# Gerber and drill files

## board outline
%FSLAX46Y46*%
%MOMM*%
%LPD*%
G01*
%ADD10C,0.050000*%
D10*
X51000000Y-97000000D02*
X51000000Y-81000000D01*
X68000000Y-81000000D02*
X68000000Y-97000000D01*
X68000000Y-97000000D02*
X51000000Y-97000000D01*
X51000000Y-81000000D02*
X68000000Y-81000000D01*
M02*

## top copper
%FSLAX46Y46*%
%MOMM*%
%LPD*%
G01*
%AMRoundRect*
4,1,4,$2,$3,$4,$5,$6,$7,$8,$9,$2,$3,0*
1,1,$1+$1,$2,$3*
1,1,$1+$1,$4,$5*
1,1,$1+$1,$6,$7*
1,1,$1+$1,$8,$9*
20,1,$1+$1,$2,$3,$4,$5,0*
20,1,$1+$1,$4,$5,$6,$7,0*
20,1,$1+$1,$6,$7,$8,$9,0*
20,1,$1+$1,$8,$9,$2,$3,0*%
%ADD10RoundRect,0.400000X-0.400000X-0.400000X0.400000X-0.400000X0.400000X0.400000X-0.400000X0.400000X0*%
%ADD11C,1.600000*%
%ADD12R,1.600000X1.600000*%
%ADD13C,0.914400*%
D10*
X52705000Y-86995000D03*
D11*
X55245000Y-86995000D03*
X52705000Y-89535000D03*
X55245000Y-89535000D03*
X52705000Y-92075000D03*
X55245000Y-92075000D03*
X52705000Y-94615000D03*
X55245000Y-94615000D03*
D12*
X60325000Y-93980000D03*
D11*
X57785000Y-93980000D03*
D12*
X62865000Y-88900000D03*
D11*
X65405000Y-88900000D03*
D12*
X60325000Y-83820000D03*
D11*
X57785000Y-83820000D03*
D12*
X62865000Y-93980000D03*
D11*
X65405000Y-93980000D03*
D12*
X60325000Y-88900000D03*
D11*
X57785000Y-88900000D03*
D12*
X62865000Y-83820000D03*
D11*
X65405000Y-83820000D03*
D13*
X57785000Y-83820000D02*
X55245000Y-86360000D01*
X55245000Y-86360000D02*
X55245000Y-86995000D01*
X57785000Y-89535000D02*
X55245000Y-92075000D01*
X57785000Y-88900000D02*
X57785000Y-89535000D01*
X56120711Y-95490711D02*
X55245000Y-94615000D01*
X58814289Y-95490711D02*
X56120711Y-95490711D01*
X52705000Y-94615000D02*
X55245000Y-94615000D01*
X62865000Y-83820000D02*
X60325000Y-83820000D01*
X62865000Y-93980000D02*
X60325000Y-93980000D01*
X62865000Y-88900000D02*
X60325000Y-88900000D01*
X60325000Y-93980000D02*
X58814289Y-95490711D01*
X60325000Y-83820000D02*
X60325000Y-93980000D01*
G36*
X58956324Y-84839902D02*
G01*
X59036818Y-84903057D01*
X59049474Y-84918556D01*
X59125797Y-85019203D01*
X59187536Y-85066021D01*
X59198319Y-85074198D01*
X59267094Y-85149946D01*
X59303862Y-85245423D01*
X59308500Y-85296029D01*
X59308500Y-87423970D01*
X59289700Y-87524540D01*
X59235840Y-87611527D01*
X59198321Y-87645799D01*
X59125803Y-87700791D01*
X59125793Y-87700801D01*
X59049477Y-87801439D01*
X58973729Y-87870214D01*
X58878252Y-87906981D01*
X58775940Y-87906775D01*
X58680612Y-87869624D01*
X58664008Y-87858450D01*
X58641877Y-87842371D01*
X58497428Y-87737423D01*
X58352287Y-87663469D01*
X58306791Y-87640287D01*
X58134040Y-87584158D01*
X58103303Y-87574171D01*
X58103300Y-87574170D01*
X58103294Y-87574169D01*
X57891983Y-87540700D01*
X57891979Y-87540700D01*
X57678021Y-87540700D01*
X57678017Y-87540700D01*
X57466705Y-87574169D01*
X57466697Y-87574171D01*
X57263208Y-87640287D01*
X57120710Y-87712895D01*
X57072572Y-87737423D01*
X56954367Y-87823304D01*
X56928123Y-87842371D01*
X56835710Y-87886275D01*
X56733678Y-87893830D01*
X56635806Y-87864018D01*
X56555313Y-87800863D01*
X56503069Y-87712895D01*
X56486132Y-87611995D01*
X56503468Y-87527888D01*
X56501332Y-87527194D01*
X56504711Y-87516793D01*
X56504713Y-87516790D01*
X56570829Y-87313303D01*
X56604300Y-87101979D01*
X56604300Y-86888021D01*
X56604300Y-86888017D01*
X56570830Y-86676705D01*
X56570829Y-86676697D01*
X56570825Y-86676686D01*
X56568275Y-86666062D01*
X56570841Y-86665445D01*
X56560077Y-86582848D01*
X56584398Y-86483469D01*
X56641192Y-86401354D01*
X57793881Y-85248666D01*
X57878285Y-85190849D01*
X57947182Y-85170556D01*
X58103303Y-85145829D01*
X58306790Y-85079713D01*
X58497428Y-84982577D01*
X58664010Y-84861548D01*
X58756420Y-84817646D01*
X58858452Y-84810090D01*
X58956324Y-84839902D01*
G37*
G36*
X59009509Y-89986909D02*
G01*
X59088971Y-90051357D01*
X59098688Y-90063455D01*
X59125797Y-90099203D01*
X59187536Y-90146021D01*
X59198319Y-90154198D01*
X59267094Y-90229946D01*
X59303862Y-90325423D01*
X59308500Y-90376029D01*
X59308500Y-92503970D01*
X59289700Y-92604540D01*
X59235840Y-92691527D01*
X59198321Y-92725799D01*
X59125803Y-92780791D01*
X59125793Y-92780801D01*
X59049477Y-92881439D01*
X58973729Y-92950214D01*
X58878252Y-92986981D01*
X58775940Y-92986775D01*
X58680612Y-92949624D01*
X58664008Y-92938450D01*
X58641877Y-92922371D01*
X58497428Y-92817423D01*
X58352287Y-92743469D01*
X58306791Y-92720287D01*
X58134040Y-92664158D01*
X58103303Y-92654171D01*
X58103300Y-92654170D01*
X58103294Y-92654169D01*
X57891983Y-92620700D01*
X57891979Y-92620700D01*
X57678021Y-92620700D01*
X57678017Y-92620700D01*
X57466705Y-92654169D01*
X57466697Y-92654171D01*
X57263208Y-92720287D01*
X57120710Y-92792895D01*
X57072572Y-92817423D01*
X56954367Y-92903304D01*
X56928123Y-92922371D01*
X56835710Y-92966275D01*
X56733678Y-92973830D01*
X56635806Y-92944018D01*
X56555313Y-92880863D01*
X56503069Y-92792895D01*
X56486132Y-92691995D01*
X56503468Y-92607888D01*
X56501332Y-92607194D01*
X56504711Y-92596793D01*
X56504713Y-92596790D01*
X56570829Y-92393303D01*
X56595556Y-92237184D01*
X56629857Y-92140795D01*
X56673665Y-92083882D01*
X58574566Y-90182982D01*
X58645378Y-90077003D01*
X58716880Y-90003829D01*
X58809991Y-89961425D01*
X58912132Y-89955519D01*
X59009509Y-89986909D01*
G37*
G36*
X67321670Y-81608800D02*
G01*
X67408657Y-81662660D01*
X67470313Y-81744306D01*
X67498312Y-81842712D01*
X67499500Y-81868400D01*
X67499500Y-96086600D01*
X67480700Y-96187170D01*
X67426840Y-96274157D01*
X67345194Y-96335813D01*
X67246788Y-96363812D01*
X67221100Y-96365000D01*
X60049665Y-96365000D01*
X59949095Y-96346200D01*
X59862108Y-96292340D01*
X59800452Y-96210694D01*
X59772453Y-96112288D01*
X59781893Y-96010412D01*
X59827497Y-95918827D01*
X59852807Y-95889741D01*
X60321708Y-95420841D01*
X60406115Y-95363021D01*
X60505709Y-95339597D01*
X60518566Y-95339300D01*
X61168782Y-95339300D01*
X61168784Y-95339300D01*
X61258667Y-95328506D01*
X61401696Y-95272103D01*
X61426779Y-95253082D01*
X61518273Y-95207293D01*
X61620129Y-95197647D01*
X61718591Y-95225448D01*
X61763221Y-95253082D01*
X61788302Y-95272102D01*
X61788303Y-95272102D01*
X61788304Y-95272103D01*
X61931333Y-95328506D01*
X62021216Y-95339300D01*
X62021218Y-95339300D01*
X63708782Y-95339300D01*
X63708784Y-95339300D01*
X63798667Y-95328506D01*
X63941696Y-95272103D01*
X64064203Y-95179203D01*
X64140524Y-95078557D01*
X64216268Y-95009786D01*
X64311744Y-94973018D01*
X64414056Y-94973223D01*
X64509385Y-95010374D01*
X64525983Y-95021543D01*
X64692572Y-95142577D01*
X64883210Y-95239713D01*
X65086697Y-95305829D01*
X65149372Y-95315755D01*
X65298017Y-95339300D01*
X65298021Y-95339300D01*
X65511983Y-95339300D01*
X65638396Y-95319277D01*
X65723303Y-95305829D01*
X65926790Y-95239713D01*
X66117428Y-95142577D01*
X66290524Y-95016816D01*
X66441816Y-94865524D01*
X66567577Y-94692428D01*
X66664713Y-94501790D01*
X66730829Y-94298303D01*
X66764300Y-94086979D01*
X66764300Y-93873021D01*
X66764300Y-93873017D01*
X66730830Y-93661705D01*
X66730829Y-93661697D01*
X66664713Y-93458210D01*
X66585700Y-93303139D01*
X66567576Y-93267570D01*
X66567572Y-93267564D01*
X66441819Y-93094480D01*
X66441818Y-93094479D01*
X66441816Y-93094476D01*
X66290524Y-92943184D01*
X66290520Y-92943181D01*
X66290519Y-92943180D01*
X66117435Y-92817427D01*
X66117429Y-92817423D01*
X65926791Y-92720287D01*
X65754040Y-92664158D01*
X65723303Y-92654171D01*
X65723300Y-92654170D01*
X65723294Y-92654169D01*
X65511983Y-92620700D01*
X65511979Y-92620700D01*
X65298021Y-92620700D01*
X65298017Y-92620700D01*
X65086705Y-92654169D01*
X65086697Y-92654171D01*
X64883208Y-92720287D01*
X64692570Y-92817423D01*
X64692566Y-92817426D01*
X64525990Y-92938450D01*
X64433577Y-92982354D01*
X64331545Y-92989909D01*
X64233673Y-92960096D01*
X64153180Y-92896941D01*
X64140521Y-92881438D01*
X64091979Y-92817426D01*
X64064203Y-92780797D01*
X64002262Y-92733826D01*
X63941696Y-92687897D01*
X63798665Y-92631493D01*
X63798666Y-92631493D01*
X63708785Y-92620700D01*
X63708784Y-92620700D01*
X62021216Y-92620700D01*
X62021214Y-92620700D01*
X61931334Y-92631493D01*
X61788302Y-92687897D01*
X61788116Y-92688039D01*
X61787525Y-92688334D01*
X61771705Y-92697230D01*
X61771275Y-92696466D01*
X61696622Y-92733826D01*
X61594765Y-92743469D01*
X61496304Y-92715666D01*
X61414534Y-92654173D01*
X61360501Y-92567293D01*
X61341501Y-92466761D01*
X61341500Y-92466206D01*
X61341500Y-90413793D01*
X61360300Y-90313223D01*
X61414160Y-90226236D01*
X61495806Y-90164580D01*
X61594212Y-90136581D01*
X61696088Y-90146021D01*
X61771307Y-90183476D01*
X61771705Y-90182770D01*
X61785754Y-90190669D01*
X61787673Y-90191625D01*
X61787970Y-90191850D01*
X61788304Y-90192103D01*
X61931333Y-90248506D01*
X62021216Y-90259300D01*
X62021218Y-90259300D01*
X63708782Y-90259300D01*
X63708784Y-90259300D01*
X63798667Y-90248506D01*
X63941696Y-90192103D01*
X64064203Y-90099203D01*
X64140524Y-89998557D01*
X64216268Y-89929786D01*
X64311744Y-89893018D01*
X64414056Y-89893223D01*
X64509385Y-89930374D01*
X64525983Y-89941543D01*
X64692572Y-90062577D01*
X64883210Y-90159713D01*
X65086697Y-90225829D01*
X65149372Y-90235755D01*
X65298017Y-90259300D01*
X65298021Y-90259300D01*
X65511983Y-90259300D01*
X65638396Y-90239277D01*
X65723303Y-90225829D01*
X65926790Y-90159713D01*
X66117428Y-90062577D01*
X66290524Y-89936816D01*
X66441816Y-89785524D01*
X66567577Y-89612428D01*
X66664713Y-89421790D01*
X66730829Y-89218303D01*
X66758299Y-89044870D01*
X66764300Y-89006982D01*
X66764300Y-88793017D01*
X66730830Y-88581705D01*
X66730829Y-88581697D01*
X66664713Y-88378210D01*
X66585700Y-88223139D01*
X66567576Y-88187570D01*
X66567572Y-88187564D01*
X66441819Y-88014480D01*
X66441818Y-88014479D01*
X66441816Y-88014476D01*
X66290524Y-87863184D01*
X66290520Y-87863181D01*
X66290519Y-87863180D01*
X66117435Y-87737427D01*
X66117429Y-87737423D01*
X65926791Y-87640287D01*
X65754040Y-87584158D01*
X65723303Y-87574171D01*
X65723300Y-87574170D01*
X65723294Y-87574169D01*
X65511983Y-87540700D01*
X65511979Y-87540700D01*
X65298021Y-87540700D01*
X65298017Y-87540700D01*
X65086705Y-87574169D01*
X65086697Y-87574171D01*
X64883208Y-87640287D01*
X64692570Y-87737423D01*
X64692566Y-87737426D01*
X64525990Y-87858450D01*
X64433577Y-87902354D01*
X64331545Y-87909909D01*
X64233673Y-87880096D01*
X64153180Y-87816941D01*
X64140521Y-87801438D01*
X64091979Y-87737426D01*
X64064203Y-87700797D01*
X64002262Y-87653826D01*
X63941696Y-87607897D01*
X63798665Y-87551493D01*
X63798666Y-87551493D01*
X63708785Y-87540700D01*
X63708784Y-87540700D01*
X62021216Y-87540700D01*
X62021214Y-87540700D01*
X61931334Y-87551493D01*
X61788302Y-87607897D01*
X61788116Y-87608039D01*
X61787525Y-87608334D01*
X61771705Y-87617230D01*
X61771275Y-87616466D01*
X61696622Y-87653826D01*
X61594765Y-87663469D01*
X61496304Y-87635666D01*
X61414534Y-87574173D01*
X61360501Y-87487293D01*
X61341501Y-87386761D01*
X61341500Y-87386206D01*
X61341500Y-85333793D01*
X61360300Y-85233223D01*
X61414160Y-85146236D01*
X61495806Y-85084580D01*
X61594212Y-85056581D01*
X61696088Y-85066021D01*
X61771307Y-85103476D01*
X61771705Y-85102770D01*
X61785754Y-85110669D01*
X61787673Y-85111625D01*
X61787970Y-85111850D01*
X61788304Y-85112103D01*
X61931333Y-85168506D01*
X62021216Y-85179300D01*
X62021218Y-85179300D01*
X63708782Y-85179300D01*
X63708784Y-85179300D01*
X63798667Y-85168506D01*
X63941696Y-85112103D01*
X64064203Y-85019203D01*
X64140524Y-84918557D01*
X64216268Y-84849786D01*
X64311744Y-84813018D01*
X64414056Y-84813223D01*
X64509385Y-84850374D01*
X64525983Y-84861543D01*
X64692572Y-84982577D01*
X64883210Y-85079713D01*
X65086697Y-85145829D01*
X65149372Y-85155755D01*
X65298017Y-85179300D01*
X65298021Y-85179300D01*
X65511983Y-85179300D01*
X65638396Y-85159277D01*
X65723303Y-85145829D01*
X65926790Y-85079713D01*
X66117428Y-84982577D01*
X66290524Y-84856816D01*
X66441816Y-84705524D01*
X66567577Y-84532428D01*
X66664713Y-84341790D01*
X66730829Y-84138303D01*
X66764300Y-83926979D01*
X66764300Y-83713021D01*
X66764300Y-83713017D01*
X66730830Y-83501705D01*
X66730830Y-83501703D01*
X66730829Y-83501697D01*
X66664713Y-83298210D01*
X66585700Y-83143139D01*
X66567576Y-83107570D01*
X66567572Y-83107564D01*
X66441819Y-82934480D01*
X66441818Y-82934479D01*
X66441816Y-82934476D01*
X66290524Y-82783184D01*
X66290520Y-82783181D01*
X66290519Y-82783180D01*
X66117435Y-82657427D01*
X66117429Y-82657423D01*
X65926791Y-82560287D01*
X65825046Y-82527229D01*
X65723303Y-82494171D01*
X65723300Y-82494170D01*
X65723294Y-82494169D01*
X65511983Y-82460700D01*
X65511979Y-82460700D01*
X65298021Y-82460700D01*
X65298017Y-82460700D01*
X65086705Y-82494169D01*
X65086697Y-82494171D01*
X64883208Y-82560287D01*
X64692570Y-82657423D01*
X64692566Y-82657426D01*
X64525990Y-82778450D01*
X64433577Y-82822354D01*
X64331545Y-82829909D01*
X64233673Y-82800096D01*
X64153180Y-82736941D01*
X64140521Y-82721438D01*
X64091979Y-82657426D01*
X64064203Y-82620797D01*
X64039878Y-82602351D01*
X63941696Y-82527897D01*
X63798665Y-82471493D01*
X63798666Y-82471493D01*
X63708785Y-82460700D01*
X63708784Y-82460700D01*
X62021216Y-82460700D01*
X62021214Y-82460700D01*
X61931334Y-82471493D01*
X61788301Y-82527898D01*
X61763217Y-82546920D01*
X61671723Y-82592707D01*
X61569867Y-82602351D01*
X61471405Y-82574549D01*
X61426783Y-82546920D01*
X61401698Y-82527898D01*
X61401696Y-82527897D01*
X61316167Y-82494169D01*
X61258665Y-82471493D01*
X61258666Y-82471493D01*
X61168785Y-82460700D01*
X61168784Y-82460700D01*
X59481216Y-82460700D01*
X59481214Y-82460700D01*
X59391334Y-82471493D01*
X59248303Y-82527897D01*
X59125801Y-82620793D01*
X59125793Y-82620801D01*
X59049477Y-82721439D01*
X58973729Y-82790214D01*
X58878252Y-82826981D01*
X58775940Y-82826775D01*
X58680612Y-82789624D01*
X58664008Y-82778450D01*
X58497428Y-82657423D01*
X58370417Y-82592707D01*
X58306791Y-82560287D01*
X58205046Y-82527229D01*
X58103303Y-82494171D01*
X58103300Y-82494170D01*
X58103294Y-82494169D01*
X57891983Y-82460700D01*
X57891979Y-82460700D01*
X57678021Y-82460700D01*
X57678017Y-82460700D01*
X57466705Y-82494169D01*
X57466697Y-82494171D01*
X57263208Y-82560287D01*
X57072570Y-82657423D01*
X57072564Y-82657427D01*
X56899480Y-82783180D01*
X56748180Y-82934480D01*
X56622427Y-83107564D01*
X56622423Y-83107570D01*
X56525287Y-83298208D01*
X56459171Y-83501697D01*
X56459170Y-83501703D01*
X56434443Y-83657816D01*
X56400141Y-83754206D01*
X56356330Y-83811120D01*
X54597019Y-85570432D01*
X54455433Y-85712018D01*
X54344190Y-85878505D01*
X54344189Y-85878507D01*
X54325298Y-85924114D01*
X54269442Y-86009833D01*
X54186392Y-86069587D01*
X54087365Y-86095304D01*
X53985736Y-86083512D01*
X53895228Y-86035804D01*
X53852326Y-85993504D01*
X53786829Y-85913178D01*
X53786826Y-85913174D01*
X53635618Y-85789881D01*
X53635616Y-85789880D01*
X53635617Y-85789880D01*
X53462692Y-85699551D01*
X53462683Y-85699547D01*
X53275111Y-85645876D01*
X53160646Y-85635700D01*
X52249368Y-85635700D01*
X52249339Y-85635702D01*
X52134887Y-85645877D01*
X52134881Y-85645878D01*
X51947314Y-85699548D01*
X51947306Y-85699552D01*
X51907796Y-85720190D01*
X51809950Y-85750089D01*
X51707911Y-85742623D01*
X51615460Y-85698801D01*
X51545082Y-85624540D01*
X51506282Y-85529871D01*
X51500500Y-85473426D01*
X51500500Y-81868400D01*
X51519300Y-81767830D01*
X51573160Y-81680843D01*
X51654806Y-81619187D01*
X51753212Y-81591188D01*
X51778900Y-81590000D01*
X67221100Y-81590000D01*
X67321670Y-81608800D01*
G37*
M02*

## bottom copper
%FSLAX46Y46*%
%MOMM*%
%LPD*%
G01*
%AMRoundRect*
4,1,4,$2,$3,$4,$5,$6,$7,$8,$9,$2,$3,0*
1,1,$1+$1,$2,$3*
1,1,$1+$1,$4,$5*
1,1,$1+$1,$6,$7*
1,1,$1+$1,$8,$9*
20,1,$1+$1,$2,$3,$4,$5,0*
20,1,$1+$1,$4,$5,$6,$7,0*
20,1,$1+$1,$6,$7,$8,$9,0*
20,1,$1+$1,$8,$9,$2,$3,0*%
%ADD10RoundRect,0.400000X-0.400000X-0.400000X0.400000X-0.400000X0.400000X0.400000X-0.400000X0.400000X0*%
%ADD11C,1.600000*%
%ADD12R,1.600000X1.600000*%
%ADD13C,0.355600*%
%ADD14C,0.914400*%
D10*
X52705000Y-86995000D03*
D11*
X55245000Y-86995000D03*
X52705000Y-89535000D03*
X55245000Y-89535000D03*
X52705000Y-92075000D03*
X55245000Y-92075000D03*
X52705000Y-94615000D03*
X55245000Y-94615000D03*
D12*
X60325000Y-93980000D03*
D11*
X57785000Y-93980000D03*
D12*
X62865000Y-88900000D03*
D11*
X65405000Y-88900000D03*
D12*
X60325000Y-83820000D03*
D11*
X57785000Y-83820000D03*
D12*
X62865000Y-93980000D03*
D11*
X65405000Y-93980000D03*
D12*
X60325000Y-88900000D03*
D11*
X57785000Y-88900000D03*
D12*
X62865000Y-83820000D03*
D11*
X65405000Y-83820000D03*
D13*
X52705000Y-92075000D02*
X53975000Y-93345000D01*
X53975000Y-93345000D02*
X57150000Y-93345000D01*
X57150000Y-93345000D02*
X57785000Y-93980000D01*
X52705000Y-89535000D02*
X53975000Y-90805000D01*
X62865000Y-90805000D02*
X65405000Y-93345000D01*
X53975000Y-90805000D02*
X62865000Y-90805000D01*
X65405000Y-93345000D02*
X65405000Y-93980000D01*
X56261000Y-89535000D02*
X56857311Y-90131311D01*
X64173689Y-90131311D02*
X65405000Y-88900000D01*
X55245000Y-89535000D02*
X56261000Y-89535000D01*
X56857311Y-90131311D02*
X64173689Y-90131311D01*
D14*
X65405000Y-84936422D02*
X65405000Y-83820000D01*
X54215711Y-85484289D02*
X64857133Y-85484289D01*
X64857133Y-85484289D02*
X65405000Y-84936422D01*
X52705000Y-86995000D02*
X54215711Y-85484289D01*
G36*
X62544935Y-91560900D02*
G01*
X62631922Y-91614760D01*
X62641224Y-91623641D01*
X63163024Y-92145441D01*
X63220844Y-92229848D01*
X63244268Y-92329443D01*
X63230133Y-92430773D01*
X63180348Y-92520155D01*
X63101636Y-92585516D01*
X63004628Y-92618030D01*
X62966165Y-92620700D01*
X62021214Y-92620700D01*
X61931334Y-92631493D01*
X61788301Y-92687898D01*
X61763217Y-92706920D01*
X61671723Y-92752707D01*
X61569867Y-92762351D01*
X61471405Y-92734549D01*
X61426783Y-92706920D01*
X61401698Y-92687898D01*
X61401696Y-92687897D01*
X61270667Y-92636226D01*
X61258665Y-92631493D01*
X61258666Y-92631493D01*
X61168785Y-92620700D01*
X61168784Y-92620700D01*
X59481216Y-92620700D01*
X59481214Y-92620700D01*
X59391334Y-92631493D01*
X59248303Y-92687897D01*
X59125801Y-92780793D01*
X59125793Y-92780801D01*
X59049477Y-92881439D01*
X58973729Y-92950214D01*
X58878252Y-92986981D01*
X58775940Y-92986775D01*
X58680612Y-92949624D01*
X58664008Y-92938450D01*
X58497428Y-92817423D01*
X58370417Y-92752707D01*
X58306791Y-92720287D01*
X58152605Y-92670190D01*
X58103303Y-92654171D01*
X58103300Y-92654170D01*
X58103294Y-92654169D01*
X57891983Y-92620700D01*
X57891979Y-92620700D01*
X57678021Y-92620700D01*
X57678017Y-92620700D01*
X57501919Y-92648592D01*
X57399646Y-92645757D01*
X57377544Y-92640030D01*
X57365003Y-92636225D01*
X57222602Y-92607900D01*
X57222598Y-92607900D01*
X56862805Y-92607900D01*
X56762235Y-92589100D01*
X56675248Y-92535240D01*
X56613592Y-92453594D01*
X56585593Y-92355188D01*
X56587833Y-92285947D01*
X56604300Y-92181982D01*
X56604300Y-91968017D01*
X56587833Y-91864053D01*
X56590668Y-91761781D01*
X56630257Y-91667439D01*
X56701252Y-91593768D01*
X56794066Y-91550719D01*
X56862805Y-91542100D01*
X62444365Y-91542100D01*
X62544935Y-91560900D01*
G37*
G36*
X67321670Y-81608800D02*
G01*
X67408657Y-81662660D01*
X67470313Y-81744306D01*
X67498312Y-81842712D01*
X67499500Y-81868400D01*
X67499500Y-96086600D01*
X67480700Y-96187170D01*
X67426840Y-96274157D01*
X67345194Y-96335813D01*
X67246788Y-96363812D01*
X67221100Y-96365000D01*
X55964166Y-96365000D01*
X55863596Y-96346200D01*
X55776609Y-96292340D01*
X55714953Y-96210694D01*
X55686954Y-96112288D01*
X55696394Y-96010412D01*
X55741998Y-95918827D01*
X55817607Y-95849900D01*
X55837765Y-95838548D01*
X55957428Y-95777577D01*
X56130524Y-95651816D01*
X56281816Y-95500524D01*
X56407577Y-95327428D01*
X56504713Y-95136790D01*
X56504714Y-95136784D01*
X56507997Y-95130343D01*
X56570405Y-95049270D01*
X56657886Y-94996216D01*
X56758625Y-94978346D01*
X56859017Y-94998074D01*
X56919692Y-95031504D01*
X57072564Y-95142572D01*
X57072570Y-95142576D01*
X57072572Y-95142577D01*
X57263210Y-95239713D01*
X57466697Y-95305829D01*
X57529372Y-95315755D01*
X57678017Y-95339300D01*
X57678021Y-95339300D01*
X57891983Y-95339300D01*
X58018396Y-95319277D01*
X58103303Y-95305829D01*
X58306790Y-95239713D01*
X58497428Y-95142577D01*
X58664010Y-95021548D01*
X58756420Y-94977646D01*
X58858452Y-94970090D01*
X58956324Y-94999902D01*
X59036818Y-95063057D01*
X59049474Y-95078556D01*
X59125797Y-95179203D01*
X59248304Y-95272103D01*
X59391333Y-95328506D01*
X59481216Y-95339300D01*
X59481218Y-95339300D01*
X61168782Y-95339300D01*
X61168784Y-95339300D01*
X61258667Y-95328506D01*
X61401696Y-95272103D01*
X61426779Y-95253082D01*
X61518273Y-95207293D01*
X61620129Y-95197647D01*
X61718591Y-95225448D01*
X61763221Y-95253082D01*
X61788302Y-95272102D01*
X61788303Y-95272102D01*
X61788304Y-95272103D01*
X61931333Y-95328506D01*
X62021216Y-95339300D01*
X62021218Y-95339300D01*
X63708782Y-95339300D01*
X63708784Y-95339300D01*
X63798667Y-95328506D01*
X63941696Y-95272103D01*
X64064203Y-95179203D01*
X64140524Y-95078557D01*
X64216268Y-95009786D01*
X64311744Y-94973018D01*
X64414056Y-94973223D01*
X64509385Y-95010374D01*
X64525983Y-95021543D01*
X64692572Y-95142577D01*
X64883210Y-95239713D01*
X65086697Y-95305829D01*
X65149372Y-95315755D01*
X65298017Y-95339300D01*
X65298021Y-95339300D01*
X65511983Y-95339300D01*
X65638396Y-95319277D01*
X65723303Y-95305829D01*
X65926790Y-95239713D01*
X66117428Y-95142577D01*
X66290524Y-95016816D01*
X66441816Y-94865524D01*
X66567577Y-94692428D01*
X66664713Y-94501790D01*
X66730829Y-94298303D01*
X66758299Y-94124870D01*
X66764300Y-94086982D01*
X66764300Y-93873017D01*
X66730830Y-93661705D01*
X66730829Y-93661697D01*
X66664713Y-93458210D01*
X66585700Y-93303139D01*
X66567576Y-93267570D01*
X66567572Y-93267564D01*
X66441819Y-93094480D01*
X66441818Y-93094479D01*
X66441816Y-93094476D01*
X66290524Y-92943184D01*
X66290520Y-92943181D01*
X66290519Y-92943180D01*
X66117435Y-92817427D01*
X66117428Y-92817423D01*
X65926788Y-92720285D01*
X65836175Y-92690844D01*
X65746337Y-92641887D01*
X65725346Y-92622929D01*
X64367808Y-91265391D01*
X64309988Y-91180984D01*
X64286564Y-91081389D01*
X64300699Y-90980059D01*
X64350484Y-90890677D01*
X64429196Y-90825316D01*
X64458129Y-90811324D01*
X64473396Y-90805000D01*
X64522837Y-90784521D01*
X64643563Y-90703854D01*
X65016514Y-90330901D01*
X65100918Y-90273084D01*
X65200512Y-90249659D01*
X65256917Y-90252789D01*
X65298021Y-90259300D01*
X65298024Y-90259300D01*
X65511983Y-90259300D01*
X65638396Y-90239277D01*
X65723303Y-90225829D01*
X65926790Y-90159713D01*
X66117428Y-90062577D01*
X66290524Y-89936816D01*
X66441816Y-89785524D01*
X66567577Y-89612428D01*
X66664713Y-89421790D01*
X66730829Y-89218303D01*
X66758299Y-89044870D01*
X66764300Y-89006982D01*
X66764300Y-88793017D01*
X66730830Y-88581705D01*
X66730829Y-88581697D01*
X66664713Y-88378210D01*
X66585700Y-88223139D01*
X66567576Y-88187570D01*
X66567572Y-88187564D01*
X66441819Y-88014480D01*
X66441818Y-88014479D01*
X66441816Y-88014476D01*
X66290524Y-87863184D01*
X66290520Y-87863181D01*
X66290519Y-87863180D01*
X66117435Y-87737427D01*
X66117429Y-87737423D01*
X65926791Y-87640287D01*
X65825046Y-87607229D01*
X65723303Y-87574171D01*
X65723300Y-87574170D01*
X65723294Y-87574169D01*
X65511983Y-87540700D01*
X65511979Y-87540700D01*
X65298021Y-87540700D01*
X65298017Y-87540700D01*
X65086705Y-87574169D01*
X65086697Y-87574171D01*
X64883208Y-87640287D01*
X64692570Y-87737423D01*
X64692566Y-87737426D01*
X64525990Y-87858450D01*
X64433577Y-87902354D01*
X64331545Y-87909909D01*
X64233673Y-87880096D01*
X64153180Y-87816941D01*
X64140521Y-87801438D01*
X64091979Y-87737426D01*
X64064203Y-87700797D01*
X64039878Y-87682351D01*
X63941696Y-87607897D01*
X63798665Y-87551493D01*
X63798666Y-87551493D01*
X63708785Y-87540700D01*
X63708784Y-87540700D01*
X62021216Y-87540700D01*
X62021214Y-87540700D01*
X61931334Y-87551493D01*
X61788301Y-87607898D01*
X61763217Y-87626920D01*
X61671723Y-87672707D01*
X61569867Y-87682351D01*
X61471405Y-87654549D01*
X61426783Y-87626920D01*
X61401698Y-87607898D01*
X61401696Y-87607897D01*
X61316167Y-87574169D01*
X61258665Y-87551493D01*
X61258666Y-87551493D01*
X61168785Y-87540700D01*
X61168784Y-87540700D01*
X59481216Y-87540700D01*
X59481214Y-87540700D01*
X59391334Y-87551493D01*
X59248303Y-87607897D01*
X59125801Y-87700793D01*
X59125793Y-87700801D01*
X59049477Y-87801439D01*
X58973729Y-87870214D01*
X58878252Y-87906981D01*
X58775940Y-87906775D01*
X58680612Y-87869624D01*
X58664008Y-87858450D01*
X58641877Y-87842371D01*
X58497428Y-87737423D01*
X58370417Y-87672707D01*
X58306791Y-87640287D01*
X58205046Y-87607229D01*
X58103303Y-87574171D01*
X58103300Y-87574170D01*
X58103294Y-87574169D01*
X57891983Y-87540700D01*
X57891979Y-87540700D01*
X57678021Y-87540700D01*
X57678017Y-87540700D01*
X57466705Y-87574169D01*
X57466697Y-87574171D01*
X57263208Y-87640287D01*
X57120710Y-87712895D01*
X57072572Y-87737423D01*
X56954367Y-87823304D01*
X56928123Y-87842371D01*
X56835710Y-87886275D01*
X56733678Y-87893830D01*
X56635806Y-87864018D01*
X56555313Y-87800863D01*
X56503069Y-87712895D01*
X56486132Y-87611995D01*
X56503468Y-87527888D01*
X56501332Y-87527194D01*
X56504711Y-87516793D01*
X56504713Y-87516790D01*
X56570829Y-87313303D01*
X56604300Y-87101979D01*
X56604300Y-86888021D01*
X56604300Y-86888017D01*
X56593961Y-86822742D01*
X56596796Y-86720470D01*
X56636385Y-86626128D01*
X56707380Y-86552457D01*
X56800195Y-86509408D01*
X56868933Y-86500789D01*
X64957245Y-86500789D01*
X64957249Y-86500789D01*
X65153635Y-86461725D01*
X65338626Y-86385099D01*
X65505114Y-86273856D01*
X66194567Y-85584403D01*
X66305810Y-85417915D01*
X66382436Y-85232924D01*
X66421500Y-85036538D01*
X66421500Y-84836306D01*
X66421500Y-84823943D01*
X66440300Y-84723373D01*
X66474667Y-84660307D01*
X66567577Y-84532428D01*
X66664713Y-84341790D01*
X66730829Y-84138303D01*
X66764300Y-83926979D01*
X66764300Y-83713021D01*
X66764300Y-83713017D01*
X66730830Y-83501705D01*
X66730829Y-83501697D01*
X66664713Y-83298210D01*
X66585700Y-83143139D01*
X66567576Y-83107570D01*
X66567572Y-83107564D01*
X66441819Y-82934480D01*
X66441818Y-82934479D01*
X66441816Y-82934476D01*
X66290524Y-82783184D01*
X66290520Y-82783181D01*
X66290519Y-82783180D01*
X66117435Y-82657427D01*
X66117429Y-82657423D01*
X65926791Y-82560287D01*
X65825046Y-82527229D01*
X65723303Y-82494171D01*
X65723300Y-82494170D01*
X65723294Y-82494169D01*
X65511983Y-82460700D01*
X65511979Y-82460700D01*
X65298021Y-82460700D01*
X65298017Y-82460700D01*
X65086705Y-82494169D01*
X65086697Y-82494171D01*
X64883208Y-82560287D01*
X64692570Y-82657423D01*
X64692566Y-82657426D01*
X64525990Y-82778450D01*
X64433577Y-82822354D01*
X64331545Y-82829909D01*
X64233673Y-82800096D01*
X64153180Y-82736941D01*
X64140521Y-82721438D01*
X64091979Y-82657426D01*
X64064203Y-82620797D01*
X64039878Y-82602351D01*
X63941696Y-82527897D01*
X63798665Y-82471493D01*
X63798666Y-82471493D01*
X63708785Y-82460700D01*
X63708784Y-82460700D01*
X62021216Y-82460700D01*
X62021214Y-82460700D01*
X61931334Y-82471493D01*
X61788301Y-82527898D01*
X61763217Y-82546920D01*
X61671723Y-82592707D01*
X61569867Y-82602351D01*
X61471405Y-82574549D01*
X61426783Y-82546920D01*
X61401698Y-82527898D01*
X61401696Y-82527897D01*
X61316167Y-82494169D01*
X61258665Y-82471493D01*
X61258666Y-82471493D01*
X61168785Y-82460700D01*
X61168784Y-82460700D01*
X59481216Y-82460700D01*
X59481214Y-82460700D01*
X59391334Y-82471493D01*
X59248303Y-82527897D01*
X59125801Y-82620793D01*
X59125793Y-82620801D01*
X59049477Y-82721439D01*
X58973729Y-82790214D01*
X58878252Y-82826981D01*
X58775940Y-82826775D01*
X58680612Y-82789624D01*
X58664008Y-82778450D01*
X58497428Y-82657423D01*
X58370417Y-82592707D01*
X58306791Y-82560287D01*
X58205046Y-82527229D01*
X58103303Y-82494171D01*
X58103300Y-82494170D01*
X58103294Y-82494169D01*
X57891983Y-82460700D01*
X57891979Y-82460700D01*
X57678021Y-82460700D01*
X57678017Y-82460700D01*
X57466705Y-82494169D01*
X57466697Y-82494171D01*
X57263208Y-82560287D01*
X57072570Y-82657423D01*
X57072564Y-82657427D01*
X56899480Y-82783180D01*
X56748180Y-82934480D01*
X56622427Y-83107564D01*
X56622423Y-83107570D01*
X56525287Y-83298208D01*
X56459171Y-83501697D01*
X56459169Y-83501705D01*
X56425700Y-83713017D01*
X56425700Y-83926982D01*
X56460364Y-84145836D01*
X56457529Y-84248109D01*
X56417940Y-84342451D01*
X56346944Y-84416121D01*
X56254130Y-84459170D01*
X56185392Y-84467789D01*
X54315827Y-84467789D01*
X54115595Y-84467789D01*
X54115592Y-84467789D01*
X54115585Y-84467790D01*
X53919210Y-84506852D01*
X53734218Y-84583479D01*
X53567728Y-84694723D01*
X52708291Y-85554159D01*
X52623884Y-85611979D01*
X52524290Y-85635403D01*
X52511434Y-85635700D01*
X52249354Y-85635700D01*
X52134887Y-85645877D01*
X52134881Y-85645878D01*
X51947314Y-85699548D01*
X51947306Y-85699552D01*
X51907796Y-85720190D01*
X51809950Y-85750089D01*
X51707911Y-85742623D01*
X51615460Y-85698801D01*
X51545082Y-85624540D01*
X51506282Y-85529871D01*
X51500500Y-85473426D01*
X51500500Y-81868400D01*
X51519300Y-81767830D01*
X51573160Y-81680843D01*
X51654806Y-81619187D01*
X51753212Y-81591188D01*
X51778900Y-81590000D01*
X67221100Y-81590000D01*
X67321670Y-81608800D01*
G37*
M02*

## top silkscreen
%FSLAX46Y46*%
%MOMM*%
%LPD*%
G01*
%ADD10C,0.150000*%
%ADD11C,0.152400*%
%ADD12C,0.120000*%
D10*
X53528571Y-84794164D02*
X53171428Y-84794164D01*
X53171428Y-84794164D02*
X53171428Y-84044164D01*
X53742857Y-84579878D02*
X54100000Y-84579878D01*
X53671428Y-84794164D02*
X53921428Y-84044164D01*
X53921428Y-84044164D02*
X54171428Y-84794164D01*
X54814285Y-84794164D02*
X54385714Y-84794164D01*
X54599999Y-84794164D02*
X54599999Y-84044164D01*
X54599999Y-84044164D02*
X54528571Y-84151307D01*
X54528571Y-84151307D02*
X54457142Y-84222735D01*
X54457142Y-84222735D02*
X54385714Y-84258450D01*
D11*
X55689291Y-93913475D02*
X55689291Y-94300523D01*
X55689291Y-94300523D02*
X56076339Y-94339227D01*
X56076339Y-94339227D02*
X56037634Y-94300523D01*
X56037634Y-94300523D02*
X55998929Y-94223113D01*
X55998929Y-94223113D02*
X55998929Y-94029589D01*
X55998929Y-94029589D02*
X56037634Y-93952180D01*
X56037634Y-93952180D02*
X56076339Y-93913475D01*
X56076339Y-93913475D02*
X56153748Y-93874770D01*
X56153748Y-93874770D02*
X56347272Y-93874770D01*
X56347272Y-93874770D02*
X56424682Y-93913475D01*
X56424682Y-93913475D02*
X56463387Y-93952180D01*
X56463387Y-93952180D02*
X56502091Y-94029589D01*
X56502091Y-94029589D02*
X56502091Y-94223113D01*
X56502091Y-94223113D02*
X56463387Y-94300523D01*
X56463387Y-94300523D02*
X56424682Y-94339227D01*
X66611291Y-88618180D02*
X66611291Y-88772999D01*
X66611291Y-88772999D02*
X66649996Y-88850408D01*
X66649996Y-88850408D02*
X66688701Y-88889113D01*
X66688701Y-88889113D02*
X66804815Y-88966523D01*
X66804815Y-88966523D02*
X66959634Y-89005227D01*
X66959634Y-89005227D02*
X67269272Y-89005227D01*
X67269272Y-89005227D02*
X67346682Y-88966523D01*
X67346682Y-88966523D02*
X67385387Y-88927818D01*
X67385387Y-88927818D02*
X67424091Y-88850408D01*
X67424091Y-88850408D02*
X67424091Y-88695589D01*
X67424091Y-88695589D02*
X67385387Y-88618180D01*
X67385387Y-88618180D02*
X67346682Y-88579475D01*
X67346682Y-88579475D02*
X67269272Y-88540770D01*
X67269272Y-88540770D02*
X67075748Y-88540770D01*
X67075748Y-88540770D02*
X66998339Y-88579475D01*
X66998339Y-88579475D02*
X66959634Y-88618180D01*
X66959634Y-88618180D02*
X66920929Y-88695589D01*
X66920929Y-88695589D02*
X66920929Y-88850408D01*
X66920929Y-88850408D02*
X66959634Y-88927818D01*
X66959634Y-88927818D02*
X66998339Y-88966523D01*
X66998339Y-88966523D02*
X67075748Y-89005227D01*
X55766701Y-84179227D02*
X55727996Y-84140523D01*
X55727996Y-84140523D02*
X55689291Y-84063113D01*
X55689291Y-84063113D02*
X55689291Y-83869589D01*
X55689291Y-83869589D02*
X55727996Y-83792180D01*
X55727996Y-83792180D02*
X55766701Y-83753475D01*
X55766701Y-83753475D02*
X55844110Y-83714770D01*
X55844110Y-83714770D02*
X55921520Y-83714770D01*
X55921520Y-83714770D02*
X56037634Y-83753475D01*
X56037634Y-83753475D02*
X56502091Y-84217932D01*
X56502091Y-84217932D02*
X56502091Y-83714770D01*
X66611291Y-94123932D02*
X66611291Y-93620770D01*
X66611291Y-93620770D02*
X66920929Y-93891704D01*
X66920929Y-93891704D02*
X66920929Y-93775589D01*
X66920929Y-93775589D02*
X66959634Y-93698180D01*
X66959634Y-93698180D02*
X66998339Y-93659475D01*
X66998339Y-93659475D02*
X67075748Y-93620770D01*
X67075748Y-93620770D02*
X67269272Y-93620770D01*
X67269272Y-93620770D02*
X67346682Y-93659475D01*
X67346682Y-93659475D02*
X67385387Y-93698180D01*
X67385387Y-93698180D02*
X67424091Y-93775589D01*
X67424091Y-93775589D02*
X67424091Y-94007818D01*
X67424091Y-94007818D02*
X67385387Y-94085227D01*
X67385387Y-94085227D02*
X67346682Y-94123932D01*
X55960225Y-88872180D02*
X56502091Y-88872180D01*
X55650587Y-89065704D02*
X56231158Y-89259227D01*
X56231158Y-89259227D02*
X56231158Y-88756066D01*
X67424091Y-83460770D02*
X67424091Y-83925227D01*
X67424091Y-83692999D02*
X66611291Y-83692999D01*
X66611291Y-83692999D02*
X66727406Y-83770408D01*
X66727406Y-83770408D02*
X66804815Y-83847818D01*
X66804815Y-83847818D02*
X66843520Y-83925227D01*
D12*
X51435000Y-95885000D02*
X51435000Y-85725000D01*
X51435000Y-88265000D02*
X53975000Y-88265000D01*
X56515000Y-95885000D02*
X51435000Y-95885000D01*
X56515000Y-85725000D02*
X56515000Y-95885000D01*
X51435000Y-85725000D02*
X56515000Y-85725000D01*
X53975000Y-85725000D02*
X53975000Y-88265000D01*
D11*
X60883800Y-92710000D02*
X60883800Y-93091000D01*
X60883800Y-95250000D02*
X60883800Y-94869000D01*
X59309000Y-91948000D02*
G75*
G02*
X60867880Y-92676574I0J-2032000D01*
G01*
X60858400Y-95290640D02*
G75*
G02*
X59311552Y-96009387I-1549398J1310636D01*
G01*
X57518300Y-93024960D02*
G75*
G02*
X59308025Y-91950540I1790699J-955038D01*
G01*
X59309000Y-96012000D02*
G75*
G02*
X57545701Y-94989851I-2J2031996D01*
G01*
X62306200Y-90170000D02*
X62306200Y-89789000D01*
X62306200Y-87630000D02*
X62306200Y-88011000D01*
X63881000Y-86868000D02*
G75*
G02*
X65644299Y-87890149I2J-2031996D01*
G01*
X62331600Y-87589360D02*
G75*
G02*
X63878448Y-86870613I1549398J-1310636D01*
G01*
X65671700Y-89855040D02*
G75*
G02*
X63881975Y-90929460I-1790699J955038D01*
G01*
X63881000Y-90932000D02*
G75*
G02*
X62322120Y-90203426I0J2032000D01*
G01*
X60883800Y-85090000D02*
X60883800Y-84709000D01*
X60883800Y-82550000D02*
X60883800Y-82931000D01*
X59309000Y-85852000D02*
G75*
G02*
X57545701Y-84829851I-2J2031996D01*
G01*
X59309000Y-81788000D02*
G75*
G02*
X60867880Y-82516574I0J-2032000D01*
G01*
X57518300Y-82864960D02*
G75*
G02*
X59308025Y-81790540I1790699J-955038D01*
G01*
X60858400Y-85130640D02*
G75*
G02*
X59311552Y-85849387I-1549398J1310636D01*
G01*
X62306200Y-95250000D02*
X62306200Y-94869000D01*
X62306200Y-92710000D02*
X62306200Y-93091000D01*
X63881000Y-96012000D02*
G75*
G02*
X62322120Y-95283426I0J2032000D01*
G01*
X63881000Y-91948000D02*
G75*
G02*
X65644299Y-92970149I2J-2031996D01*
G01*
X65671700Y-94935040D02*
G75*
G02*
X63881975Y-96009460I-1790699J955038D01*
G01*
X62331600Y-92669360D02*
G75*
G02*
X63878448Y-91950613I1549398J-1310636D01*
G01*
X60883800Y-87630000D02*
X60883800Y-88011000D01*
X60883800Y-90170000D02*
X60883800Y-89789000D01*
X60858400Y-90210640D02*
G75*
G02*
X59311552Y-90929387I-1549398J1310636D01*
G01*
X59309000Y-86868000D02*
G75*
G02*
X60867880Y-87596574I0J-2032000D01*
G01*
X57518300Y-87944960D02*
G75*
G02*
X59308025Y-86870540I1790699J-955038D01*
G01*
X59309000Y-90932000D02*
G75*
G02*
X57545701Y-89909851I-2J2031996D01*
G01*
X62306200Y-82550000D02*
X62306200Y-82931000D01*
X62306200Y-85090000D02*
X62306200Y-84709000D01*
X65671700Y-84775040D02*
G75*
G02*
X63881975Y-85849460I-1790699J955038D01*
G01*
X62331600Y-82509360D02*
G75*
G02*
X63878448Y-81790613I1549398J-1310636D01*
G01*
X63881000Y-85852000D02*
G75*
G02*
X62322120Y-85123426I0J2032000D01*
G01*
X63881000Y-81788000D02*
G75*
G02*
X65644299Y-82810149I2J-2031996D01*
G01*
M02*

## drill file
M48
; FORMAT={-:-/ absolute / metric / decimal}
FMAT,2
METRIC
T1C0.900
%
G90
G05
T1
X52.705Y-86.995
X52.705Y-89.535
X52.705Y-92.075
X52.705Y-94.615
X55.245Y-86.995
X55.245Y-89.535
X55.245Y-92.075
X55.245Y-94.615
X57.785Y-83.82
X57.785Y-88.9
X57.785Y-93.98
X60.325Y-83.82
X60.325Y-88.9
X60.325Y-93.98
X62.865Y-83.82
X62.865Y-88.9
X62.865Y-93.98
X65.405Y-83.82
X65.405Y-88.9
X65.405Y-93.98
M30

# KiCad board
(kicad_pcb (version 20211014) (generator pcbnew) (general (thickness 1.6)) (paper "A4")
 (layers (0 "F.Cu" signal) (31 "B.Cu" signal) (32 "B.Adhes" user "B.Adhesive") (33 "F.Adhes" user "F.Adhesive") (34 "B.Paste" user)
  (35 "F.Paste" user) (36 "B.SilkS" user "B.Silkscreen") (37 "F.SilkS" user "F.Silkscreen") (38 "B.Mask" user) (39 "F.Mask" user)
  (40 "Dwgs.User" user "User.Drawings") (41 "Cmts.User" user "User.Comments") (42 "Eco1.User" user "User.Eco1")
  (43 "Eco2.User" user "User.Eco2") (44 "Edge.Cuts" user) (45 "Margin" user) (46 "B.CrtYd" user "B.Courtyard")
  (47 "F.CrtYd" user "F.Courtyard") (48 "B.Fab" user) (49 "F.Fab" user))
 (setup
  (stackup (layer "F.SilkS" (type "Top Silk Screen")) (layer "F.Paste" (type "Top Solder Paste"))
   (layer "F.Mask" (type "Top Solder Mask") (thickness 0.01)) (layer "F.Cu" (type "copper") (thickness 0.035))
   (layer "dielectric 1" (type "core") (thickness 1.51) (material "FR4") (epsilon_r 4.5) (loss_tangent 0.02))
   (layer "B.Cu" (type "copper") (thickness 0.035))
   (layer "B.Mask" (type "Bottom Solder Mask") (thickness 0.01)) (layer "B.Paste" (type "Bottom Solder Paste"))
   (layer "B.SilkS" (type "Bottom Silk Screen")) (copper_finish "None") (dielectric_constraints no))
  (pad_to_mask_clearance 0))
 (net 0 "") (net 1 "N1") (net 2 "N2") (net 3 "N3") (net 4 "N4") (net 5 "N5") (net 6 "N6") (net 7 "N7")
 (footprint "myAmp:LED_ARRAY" (layer "F.Cu") (at 53.975 90.805)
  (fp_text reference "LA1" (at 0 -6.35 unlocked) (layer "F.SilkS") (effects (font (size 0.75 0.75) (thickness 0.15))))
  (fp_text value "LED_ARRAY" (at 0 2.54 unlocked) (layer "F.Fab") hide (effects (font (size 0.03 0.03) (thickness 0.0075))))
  (fp_line (start -2.54 5.08) (end -2.54 -5.08) (layer "F.SilkS") (width 0.12))
  (fp_line (start -2.54 -2.54) (end 0 -2.54) (layer "F.SilkS") (width 0.12))
  (fp_line (start 2.54 5.08) (end -2.54 5.08) (layer "F.SilkS") (width 0.12))
  (fp_line (start 2.54 -5.08) (end 2.54 5.08) (layer "F.SilkS") (width 0.12))
  (fp_line (start -2.54 -5.08) (end 2.54 -5.08) (layer "F.SilkS") (width 0.12))
  (fp_line (start 0 -5.08) (end 0 -2.54) (layer "F.SilkS") (width 0.12))
  (pad "1" thru_hole roundrect (at -1.27 -3.81) (size 1.6 1.6) (drill 0.9) (layers *.Cu *.Mask) (roundrect_rratio 0.25) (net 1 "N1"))
  (pad "2" thru_hole circle (at 1.27 -3.81) (size 1.6 1.6) (drill 0.9) (layers *.Cu *.Mask) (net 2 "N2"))
  (pad "3" thru_hole circle (at -1.27 -1.27) (size 1.6 1.6) (drill 0.9) (layers *.Cu *.Mask) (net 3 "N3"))
  (pad "4" thru_hole circle (at 1.27 -1.27) (size 1.6 1.6) (drill 0.9) (layers *.Cu *.Mask) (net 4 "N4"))
  (pad "5" thru_hole circle (at -1.27 1.27) (size 1.6 1.6) (drill 0.9) (layers *.Cu *.Mask) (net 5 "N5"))
  (pad "6" thru_hole circle (at 1.27 1.27) (size 1.6 1.6) (drill 0.9) (layers *.Cu *.Mask) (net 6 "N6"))
  (pad "7" thru_hole circle (at -1.27 3.81) (size 1.6 1.6) (drill 0.9) (layers *.Cu *.Mask) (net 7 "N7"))
  (pad "8" thru_hole circle (at 1.27 3.81) (size 1.6 1.6) (drill 0.9) (layers *.Cu *.Mask) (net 7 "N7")))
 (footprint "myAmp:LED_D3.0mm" (layer "F.Cu") (at 59.055 93.98)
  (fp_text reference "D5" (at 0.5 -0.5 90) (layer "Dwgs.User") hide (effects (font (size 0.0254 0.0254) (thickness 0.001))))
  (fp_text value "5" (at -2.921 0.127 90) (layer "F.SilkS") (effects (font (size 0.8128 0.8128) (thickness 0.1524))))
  (fp_line (start 1.8288 -1.27) (end 1.8288 -0.889) (layer "F.SilkS") (width 0.1524))
  (fp_line (start 1.8288 1.27) (end 1.8288 0.889) (layer "F.SilkS") (width 0.1524))
  (fp_arc (start 0.254 -2.032) (mid 1.114367 -1.840867) (end 1.81288 -1.303426) (layer "F.SilkS") (width 0.1524))
  (fp_arc (start 1.8034 1.31064) (mid 1.109154 1.840416) (end 0.256552 2.029387) (layer "F.SilkS") (width 0.1524))
  (fp_arc (start -1.5367 -0.95504) (mid -0.790567 -1.739997) (end 0.253025 -2.02946) (layer "F.SilkS") (width 0.1524))
  (fp_arc (start 0.254 2.032) (mid -0.76507 1.757988) (end -1.509299 1.009851) (layer "F.SilkS") (width 0.1524))
  (pad "1" thru_hole rect locked (at 1.27 0) (size 1.6 1.6) (drill 0.9) (layers *.Cu *.Mask) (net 7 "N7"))
  (pad "2" thru_hole circle locked (at -1.27 0) (size 1.6 1.6) (drill 0.9) (layers *.Cu *.Mask) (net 5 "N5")))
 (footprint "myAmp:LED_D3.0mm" (layer "F.Cu") (at 64.135 88.9 180)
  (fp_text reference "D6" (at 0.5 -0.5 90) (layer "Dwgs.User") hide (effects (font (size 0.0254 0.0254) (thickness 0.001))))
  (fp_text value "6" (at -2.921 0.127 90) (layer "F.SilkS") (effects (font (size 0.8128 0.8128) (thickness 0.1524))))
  (fp_line (start 1.8288 -1.27) (end 1.8288 -0.889) (layer "F.SilkS") (width 0.1524))
  (fp_line (start 1.8288 1.27) (end 1.8288 0.889) (layer "F.SilkS") (width 0.1524))
  (fp_arc (start 0.254 2.032) (mid -0.76507 1.757988) (end -1.509299 1.009851) (layer "F.SilkS") (width 0.1524))
  (fp_arc (start 1.8034 1.31064) (mid 1.109154 1.840416) (end 0.256552 2.029387) (layer "F.SilkS") (width 0.1524))
  (fp_arc (start -1.5367 -0.95504) (mid -0.790567 -1.739997) (end 0.253025 -2.02946) (layer "F.SilkS") (width 0.1524))
  (fp_arc (start 0.254 -2.032) (mid 1.114367 -1.840867) (end 1.81288 -1.303426) (layer "F.SilkS") (width 0.1524))
  (pad "1" thru_hole rect locked (at 1.27 0 180) (size 1.6 1.6) (drill 0.9) (layers *.Cu *.Mask) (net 7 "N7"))
  (pad "2" thru_hole circle locked (at -1.27 0 180) (size 1.6 1.6) (drill 0.9) (layers *.Cu *.Mask) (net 4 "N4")))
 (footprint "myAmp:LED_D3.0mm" (layer "F.Cu") (at 59.055 83.82)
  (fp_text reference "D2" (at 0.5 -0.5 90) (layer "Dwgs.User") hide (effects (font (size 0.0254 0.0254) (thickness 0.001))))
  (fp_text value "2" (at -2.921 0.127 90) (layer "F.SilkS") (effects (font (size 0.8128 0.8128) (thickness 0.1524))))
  (fp_line (start 1.8288 1.27) (end 1.8288 0.889) (layer "F.SilkS") (width 0.1524))
  (fp_line (start 1.8288 -1.27) (end 1.8288 -0.889) (layer "F.SilkS") (width 0.1524))
  (fp_arc (start 0.254 2.032) (mid -0.76507 1.757988) (end -1.509299 1.009851) (layer "F.SilkS") (width 0.1524))
  (fp_arc (start 0.254 -2.032) (mid 1.114367 -1.840867) (end 1.81288 -1.303426) (layer "F.SilkS") (width 0.1524))
  (fp_arc (start -1.5367 -0.95504) (mid -0.790567 -1.739997) (end 0.253025 -2.02946) (layer "F.SilkS") (width 0.1524))
  (fp_arc (start 1.8034 1.31064) (mid 1.109154 1.840416) (end 0.256552 2.029387) (layer "F.SilkS") (width 0.1524))
  (pad "1" thru_hole rect locked (at 1.27 0) (size 1.6 1.6) (drill 0.9) (layers *.Cu *.Mask) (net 7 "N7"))
  (pad "2" thru_hole circle locked (at -1.27 0) (size 1.6 1.6) (drill 0.9) (layers *.Cu *.Mask) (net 2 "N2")))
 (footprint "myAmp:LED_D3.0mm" (layer "F.Cu") (at 64.135 93.98 180)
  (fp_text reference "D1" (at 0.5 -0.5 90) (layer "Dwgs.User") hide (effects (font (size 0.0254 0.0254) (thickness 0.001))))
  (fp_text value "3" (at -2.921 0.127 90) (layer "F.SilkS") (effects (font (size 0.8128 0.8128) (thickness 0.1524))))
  (fp_line (start 1.8288 -1.27) (end 1.8288 -0.889) (layer "F.SilkS") (width 0.1524))
  (fp_line (start 1.8288 1.27) (end 1.8288 0.889) (layer "F.SilkS") (width 0.1524))
  (fp_arc (start 0.254 -2.032) (mid 1.114367 -1.840867) (end 1.81288 -1.303426) (layer "F.SilkS") (width 0.1524))
  (fp_arc (start 0.254 2.032) (mid -0.76507 1.757988) (end -1.509299 1.009851) (layer "F.SilkS") (width 0.1524))
  (fp_arc (start -1.5367 -0.95504) (mid -0.790567 -1.739997) (end 0.253025 -2.02946) (layer "F.SilkS") (width 0.1524))
  (fp_arc (start 1.8034 1.31064) (mid 1.109154 1.840416) (end 0.256552 2.029387) (layer "F.SilkS") (width 0.1524))
  (pad "1" thru_hole rect locked (at 1.27 0 180) (size 1.6 1.6) (drill 0.9) (layers *.Cu *.Mask) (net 7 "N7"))
  (pad "2" thru_hole circle locked (at -1.27 0 180) (size 1.6 1.6) (drill 0.9) (layers *.Cu *.Mask) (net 3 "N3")))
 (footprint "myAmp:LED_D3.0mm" (layer "F.Cu") (at 59.055 88.9)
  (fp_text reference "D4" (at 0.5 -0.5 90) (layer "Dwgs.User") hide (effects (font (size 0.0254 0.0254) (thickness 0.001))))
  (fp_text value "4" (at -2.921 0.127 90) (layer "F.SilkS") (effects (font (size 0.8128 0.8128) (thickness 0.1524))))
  (fp_line (start 1.8288 -1.27) (end 1.8288 -0.889) (layer "F.SilkS") (width 0.1524))
  (fp_line (start 1.8288 1.27) (end 1.8288 0.889) (layer "F.SilkS") (width 0.1524))
  (fp_arc (start 1.8034 1.31064) (mid 1.109154 1.840416) (end 0.256552 2.029387) (layer "F.SilkS") (width 0.1524))
  (fp_arc (start 0.254 -2.032) (mid 1.114367 -1.840867) (end 1.81288 -1.303426) (layer "F.SilkS") (width 0.1524))
  (fp_arc (start -1.5367 -0.95504) (mid -0.790567 -1.739997) (end 0.253025 -2.02946) (layer "F.SilkS") (width 0.1524))
  (fp_arc (start 0.254 2.032) (mid -0.76507 1.757988) (end -1.509299 1.009851) (layer "F.SilkS") (width 0.1524))
  (pad "1" thru_hole rect locked (at 1.27 0) (size 1.6 1.6) (drill 0.9) (layers *.Cu *.Mask) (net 7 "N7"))
  (pad "2" thru_hole circle locked (at -1.27 0) (size 1.6 1.6) (drill 0.9) (layers *.Cu *.Mask) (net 6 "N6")))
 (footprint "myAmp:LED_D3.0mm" (layer "F.Cu") (at 64.135 83.82 180)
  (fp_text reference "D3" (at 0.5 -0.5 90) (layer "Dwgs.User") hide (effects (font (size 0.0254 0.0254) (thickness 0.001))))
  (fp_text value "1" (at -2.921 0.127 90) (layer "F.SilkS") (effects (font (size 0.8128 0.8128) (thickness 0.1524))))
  (fp_line (start 1.8288 1.27) (end 1.8288 0.889) (layer "F.SilkS") (width 0.1524))
  (fp_line (start 1.8288 -1.27) (end 1.8288 -0.889) (layer "F.SilkS") (width 0.1524))
  (fp_arc (start -1.5367 -0.95504) (mid -0.790567 -1.739997) (end 0.253025 -2.02946) (layer "F.SilkS") (width 0.1524))
  (fp_arc (start 1.8034 1.31064) (mid 1.109154 1.840416) (end 0.256552 2.029387) (layer "F.SilkS") (width 0.1524))
  (fp_arc (start 0.254 -2.032) (mid 1.114367 -1.840867) (end 1.81288 -1.303426) (layer "F.SilkS") (width 0.1524))
  (fp_arc (start 0.254 2.032) (mid -0.76507 1.757988) (end -1.509299 1.009851) (layer "F.SilkS") (width 0.1524))
  (pad "1" thru_hole rect locked (at 1.27 0 180) (size 1.6 1.6) (drill 0.9) (layers *.Cu *.Mask) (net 7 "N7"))
  (pad "2" thru_hole circle locked (at -1.27 0 180) (size 1.6 1.6) (drill 0.9) (layers *.Cu *.Mask) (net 1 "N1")))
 (gr_line (start 51 97) (end 51 81) (layer "Edge.Cuts") (width 0.05))
 (gr_line (start 68 81) (end 68 97) (layer "Edge.Cuts") (width 0.05))
 (gr_line (start 68 97) (end 51 97) (layer "Edge.Cuts") (width 0.05))
 (gr_line (start 51 81) (end 68 81) (layer "Edge.Cuts") (width 0.05))
 (segment (start 57.785 83.82) (end 55.245 86.36) (width 0.9144) (layer "F.Cu") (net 2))
 (segment (start 55.245 86.36) (end 55.245 86.995) (width 0.9144) (layer "F.Cu") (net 2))
 (segment (start 57.785 89.535) (end 55.245 92.075) (width 0.9144) (layer "F.Cu") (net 6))
 (segment (start 57.785 88.9) (end 57.785 89.535) (width 0.9144) (layer "F.Cu") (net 6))
 (segment (start 52.705 92.075) (end 53.975 93.345) (width 0.3556) (layer "B.Cu") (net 5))
 (segment (start 53.975 93.345) (end 57.15 93.345) (width 0.3556) (layer "B.Cu") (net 5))
 (segment (start 57.15 93.345) (end 57.785 93.98) (width 0.3556) (layer "B.Cu") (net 5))
 (segment (start 52.705 89.535) (end 53.975 90.805) (width 0.3556) (layer "B.Cu") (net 3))
 (segment (start 62.865 90.805) (end 65.405 93.345) (width 0.3556) (layer "B.Cu") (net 3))
 (segment (start 53.975 90.805) (end 62.865 90.805) (width 0.3556) (layer "B.Cu") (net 3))
 (segment (start 65.405 93.345) (end 65.405 93.98) (width 0.3556) (layer "B.Cu") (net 3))
 (segment (start 56.261 89.535) (end 56.857311 90.131311) (width 0.3556) (layer "B.Cu") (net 4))
 (segment (start 64.173689 90.131311) (end 65.405 88.9) (width 0.3556) (layer "B.Cu") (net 4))
 (segment (start 55.245 89.535) (end 56.261 89.535) (width 0.3556) (layer "B.Cu") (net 4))
 (segment (start 56.857311 90.131311) (end 64.173689 90.131311) (width 0.3556) (layer "B.Cu") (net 4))
 (segment (start 56.120711 95.490711) (end 55.245 94.615) (width 0.9144) (layer "F.Cu") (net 7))
 (segment (start 58.814289 95.490711) (end 56.120711 95.490711) (width 0.9144) (layer "F.Cu") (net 7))
 (segment (start 52.705 94.615) (end 55.245 94.615) (width 0.9144) (layer "F.Cu") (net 7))
 (segment (start 62.865 83.82) (end 60.325 83.82) (width 0.9144) (layer "F.Cu") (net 7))
 (segment (start 62.865 93.98) (end 60.325 93.98) (width 0.9144) (layer "F.Cu") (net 7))
 (segment (start 62.865 88.9) (end 60.325 88.9) (width 0.9144) (layer "F.Cu") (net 7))
 (segment (start 60.325 93.98) (end 58.814289 95.490711) (width 0.9144) (layer "F.Cu") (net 7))
 (segment (start 60.325 83.82) (end 60.325 93.98) (width 0.9144) (layer "F.Cu") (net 7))
 (segment (start 65.405 84.936422) (end 65.405 83.82) (width 0.9144) (layer "B.Cu") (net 1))
 (segment (start 54.215711 85.484289) (end 64.857133 85.484289) (width 0.9144) (layer "B.Cu") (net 1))
 (segment (start 64.857133 85.484289) (end 65.405 84.936422) (width 0.9144) (layer "B.Cu") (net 1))
 (segment (start 52.705 86.995) (end 54.215711 85.484289) (width 0.9144) (layer "B.Cu") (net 1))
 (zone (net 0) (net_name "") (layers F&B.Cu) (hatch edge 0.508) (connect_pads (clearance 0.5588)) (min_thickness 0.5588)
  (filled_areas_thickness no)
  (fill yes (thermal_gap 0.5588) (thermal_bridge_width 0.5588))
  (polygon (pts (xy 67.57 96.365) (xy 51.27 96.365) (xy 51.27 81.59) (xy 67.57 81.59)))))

